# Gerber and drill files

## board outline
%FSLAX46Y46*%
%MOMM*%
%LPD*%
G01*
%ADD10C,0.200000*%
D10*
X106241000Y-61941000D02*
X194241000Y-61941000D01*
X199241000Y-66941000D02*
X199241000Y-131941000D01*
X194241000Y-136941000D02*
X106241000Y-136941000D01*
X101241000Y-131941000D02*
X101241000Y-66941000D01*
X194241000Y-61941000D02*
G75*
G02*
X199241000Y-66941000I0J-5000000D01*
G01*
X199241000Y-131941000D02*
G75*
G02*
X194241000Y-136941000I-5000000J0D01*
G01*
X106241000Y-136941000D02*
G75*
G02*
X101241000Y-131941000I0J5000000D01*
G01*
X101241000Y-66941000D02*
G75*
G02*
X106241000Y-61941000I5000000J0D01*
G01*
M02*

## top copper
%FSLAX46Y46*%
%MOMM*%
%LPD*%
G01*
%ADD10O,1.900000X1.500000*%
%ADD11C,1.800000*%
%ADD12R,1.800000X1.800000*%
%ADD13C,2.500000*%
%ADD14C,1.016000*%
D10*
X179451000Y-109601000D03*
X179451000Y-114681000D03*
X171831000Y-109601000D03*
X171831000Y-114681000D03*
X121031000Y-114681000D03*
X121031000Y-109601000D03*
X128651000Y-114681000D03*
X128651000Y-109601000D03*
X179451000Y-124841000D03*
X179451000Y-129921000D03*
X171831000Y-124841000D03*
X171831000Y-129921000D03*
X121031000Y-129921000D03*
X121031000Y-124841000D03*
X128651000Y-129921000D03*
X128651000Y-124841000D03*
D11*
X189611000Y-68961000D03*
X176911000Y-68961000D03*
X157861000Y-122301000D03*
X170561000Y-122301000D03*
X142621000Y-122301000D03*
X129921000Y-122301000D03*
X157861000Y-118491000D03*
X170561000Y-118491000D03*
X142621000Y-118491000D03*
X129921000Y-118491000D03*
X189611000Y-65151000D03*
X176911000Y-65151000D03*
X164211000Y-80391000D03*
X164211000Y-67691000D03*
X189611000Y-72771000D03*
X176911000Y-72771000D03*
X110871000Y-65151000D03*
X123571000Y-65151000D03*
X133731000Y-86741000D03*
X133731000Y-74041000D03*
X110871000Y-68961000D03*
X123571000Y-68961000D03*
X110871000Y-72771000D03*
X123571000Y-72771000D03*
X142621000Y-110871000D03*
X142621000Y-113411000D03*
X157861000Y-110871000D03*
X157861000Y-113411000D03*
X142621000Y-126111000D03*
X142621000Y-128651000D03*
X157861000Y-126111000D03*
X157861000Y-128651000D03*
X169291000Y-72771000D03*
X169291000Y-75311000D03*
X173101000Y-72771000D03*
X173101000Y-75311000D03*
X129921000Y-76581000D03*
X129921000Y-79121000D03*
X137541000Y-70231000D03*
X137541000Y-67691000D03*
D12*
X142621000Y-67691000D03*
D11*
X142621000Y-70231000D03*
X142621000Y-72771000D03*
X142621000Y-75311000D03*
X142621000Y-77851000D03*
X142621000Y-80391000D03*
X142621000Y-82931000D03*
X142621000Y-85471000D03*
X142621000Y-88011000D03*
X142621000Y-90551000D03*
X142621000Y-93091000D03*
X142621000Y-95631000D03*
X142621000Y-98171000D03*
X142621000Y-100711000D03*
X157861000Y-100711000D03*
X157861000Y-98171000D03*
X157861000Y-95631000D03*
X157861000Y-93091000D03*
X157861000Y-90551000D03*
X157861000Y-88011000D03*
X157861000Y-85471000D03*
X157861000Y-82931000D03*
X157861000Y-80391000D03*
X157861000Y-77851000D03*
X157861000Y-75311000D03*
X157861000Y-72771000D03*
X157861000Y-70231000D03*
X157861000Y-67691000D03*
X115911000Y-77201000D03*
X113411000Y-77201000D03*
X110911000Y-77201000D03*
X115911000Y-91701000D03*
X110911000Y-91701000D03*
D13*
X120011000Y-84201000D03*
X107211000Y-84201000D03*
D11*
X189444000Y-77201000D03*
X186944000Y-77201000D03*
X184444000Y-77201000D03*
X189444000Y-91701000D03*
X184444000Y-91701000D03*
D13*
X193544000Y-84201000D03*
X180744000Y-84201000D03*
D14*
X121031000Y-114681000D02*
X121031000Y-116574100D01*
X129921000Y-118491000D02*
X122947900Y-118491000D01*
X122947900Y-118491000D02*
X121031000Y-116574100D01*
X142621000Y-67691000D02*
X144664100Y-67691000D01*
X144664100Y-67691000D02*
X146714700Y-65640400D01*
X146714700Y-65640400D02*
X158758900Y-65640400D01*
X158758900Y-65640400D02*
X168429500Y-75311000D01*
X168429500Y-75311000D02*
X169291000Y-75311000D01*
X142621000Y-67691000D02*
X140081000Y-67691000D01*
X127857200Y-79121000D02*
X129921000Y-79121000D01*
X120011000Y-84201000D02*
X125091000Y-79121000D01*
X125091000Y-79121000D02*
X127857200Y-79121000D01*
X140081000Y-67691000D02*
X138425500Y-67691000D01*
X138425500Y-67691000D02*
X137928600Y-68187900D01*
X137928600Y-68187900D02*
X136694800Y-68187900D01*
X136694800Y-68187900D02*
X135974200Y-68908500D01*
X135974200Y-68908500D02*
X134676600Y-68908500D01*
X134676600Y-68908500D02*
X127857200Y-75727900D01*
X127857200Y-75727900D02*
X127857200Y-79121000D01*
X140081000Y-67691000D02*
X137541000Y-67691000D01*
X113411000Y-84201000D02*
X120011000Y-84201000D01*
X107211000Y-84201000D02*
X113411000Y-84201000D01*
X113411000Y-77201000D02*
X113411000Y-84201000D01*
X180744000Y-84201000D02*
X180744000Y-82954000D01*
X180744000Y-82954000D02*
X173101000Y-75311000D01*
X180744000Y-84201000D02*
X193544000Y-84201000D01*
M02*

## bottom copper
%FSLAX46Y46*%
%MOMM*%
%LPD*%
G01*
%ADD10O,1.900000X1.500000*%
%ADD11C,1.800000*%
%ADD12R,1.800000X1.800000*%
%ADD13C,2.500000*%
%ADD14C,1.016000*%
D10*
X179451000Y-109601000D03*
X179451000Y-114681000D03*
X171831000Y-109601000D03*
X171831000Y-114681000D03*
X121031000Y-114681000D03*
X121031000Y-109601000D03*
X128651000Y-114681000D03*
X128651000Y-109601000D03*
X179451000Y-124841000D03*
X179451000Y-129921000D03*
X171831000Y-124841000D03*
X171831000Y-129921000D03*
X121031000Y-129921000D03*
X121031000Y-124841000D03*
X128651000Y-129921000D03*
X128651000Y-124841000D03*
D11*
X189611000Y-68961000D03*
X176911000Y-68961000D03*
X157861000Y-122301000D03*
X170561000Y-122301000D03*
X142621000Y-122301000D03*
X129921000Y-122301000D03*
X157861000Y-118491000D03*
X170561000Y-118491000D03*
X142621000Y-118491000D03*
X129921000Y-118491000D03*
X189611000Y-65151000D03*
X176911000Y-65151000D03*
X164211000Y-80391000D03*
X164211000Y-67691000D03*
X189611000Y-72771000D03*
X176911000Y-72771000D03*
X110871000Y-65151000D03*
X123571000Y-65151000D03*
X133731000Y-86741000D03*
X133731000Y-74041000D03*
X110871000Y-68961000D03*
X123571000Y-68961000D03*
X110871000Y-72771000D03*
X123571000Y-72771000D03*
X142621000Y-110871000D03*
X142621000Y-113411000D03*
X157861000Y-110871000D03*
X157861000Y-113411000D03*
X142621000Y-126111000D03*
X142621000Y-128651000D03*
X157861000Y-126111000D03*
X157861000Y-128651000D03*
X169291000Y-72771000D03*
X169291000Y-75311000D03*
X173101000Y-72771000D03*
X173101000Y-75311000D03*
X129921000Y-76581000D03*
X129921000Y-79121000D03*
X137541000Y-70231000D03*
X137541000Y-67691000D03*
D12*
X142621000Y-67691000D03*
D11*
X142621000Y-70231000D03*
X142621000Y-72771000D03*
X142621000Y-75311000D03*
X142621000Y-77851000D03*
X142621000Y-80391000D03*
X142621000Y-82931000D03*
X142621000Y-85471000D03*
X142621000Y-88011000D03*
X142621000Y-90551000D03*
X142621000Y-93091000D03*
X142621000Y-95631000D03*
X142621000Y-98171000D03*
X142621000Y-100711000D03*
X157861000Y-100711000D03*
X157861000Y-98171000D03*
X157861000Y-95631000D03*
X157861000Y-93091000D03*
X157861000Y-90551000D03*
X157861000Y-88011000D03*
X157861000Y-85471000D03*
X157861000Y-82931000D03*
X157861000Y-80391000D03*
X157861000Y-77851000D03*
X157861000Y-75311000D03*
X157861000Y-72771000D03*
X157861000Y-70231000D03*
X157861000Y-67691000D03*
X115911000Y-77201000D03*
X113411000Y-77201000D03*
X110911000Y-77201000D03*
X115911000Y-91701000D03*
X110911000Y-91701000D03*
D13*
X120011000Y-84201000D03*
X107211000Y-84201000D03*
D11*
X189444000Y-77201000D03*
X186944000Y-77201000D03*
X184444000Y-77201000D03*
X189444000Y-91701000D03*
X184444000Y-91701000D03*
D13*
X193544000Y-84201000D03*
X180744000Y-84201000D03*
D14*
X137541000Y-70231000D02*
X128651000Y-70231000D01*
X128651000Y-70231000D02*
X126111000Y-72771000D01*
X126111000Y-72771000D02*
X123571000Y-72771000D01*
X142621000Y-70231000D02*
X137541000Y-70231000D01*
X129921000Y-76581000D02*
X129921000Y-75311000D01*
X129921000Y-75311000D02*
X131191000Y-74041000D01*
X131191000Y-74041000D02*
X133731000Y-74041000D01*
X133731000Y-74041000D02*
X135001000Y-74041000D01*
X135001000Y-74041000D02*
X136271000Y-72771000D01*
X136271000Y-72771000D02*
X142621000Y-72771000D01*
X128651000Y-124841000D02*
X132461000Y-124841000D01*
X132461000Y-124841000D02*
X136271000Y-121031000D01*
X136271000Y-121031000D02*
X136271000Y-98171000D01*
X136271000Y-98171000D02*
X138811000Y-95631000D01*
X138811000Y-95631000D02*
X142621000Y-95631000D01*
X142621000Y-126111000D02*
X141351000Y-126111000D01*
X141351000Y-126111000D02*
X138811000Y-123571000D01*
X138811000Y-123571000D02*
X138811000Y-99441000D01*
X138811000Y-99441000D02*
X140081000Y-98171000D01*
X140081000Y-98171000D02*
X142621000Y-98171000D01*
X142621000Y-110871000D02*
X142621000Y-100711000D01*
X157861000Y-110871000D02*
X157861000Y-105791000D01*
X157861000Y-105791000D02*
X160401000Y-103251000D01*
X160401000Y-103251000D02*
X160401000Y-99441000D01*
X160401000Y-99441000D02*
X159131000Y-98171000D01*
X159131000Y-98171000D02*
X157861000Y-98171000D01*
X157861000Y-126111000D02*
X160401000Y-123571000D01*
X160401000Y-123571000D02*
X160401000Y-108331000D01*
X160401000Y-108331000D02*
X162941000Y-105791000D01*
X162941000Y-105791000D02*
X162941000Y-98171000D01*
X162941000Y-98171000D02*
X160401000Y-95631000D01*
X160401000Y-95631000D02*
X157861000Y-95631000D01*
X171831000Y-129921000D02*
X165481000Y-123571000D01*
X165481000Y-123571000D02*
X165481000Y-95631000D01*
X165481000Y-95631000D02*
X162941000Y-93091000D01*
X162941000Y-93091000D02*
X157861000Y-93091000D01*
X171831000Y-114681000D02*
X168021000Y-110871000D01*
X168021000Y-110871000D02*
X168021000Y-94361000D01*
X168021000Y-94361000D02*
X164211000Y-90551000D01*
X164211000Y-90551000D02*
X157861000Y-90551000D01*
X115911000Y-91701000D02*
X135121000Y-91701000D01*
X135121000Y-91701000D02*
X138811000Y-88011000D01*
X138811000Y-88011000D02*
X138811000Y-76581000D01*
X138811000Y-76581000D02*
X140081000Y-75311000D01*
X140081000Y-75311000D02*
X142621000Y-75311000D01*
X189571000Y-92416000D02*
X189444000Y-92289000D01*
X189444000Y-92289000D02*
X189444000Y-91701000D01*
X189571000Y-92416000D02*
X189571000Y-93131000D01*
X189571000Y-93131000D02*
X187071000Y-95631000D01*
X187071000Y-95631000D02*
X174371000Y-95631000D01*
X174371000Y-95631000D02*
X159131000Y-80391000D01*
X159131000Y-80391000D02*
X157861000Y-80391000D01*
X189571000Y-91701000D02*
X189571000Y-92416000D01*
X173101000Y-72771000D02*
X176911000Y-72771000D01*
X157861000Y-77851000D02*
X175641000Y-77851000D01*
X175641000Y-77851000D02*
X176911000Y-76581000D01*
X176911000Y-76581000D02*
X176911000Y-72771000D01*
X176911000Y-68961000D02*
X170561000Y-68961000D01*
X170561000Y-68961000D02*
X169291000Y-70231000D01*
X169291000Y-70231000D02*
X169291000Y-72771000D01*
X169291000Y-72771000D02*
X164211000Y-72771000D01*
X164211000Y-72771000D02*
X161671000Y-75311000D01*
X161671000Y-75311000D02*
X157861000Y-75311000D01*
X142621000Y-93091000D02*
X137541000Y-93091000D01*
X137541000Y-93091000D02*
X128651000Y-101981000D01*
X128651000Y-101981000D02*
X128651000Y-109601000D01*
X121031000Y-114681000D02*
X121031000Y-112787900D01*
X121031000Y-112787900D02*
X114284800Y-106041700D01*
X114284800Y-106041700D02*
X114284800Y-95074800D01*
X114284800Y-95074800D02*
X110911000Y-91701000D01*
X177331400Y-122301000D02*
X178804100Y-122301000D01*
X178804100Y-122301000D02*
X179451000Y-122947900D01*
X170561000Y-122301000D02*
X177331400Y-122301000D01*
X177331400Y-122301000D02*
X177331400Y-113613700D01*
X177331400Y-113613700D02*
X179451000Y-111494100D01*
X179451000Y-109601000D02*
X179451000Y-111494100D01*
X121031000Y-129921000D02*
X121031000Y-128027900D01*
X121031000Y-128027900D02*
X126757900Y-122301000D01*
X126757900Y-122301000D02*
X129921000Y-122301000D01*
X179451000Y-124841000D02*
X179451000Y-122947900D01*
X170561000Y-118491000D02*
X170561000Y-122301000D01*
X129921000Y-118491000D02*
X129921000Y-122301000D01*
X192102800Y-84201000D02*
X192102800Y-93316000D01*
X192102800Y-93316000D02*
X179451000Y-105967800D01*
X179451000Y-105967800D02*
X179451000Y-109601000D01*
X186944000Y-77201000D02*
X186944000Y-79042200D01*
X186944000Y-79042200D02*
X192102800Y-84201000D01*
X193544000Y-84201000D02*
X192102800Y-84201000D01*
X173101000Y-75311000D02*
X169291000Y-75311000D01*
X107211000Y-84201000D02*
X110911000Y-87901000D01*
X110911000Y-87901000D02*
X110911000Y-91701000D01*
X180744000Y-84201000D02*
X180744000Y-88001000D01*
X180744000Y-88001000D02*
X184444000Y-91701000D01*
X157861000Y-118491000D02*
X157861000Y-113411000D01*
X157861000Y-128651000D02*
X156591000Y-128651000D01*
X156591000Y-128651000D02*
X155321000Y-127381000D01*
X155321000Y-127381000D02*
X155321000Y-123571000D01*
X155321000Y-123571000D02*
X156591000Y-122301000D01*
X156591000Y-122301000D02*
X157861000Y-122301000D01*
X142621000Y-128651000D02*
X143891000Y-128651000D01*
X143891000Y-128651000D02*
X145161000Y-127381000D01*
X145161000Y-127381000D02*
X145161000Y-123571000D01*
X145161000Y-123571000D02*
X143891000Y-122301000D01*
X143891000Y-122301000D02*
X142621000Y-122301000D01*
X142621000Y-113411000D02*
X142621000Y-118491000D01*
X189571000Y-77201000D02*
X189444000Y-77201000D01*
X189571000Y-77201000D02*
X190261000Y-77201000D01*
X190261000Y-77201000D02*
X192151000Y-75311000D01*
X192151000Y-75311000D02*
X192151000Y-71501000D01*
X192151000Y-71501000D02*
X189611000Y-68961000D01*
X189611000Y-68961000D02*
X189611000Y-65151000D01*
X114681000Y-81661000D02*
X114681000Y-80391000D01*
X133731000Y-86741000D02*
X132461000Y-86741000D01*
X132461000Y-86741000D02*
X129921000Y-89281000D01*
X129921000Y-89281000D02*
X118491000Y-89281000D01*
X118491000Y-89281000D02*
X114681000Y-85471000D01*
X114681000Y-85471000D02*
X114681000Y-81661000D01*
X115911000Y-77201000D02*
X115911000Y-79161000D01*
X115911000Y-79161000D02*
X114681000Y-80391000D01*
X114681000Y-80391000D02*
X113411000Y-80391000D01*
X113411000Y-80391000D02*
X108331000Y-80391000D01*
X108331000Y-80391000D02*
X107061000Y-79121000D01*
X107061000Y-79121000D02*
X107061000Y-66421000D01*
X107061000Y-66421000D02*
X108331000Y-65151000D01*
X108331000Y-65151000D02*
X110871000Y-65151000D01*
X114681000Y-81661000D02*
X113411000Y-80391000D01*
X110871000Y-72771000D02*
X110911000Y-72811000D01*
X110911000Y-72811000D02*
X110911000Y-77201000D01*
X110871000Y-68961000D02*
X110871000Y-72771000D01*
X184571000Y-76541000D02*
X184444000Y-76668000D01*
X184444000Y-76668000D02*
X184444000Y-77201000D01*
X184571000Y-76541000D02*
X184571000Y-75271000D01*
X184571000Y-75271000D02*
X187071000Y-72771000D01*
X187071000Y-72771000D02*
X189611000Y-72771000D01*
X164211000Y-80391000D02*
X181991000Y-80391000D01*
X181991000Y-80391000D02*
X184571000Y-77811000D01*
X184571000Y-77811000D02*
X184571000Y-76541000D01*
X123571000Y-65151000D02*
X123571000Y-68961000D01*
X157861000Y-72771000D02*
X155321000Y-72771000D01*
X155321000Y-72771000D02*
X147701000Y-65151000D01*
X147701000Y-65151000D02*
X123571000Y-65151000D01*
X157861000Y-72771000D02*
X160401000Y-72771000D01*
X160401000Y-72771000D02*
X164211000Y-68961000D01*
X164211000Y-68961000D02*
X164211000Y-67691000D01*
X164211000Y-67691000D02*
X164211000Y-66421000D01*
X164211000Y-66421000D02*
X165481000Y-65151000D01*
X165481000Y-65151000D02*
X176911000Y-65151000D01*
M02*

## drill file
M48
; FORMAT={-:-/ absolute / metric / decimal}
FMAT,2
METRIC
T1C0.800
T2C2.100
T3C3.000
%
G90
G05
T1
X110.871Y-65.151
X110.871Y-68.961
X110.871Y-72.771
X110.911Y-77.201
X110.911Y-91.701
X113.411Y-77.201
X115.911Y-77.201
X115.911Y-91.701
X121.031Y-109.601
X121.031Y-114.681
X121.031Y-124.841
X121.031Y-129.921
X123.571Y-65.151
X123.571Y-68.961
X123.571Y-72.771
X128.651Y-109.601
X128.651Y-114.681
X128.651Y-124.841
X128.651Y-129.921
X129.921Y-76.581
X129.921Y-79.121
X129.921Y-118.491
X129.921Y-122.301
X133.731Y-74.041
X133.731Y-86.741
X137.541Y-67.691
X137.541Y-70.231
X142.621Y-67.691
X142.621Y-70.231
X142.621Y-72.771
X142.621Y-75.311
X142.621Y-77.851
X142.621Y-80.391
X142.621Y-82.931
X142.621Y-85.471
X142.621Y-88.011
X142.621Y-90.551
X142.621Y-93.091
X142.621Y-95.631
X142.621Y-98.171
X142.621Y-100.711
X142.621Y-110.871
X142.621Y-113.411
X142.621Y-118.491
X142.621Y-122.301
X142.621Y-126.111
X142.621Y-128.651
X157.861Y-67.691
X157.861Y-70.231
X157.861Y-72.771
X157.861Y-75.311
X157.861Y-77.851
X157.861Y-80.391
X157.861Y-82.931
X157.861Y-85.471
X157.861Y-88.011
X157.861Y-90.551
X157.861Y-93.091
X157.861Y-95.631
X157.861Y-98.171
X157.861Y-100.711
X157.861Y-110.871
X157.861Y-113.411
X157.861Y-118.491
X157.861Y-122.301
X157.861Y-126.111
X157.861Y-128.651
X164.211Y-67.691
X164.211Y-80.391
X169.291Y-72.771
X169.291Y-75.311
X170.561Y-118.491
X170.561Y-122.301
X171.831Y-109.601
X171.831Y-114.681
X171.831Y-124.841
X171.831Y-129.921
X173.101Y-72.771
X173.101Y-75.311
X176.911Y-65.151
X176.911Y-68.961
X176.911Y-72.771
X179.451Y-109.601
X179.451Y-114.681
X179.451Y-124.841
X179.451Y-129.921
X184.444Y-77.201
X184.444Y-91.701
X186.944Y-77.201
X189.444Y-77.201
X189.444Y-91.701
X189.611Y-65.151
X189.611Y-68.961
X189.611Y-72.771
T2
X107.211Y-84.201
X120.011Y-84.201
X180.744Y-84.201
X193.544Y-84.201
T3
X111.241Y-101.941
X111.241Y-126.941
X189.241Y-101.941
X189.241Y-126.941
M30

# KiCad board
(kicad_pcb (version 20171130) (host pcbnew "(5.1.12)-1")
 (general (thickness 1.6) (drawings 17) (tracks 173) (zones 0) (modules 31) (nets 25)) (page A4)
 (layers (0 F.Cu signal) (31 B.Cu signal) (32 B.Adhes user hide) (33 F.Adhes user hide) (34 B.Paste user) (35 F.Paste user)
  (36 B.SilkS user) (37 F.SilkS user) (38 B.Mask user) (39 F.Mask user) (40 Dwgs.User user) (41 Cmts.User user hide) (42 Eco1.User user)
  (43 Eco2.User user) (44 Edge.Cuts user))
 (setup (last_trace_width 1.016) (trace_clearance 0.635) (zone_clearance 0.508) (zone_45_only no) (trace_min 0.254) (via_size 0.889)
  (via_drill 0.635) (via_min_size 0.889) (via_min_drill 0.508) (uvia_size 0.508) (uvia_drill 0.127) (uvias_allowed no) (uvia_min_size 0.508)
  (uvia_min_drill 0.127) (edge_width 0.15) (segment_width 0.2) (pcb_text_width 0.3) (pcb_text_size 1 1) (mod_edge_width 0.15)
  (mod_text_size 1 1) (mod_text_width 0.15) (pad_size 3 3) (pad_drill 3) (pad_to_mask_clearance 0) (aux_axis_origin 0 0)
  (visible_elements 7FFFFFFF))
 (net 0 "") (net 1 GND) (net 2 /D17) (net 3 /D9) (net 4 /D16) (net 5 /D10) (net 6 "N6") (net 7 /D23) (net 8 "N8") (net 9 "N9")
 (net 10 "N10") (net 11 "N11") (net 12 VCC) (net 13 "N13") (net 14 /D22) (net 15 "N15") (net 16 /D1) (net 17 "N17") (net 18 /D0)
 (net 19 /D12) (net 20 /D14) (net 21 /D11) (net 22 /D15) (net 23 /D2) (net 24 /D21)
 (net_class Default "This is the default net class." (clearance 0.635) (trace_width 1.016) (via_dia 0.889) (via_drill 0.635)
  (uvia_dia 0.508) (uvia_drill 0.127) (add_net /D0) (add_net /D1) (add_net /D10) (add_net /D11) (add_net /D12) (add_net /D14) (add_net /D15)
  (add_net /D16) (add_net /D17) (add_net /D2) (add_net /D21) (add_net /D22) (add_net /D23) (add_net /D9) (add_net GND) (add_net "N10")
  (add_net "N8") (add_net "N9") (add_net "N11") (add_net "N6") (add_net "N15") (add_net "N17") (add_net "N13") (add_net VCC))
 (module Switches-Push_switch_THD (layer F.Cu) (at 175.641 112.141 180)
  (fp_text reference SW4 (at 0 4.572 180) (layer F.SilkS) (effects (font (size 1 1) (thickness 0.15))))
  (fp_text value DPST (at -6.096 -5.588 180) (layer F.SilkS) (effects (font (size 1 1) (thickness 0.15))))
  (pad 2 thru_hole oval (at -3.81 2.54 180) (size 1.9 1.5) (drill 0.8) (layers *.Cu *.Mask F.SilkS) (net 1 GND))
  (pad 1 thru_hole oval (at -3.81 -2.54 180) (size 1.9 1.5) (drill 0.8) (layers *.Cu *.Mask F.SilkS))
  (pad 4 thru_hole oval (at 3.81 2.54 180) (size 1.9 1.5) (drill 0.8) (layers *.Cu *.Mask F.SilkS))
  (pad 3 thru_hole oval (at 3.81 -2.54 180) (size 1.9 1.5) (drill 0.8) (layers *.Cu *.Mask F.SilkS) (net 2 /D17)))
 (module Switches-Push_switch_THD (layer F.Cu) (at 124.841 112.141)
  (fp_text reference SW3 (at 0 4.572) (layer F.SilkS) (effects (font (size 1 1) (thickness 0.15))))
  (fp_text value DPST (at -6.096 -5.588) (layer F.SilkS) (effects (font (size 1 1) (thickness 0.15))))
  (pad 2 thru_hole oval (at -3.81 2.54) (size 1.9 1.5) (drill 0.8) (layers *.Cu *.Mask F.SilkS) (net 1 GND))
  (pad 1 thru_hole oval (at -3.81 -2.54) (size 1.9 1.5) (drill 0.8) (layers *.Cu *.Mask F.SilkS))
  (pad 4 thru_hole oval (at 3.81 2.54) (size 1.9 1.5) (drill 0.8) (layers *.Cu *.Mask F.SilkS))
  (pad 3 thru_hole oval (at 3.81 -2.54) (size 1.9 1.5) (drill 0.8) (layers *.Cu *.Mask F.SilkS) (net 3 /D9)))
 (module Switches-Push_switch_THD (layer F.Cu) (at 175.641 127.381 180)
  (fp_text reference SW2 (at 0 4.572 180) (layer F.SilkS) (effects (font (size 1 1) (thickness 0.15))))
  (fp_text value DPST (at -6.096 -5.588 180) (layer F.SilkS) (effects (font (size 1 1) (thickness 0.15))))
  (pad 2 thru_hole oval (at -3.81 2.54 180) (size 1.9 1.5) (drill 0.8) (layers *.Cu *.Mask F.SilkS) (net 1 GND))
  (pad 1 thru_hole oval (at -3.81 -2.54 180) (size 1.9 1.5) (drill 0.8) (layers *.Cu *.Mask F.SilkS))
  (pad 4 thru_hole oval (at 3.81 2.54 180) (size 1.9 1.5) (drill 0.8) (layers *.Cu *.Mask F.SilkS))
  (pad 3 thru_hole oval (at 3.81 -2.54 180) (size 1.9 1.5) (drill 0.8) (layers *.Cu *.Mask F.SilkS) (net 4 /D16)))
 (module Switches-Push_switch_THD (layer F.Cu) (at 124.841 127.381)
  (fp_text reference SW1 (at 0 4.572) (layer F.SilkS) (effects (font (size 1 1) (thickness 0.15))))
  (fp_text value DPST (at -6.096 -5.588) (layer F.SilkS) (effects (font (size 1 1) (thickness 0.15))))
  (pad 2 thru_hole oval (at -3.81 2.54) (size 1.9 1.5) (drill 0.8) (layers *.Cu *.Mask F.SilkS) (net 1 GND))
  (pad 1 thru_hole oval (at -3.81 -2.54) (size 1.9 1.5) (drill 0.8) (layers *.Cu *.Mask F.SilkS))
  (pad 4 thru_hole oval (at 3.81 2.54) (size 1.9 1.5) (drill 0.8) (layers *.Cu *.Mask F.SilkS))
  (pad 3 thru_hole oval (at 3.81 -2.54) (size 1.9 1.5) (drill 0.8) (layers *.Cu *.Mask F.SilkS) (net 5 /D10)))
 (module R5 (layer F.Cu) (at 183.261 68.961 180) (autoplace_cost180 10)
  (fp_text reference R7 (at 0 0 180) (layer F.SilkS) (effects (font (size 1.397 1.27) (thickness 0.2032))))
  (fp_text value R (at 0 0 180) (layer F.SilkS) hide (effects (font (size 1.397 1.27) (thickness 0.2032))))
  (pad 1 thru_hole circle (at -6.35 0 180) (size 1.8 1.8) (drill 0.8) (layers *.Cu *.Mask F.SilkS) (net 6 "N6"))
  (pad 2 thru_hole circle (at 6.35 0 180) (size 1.8 1.8) (drill 0.8) (layers *.Cu *.Mask F.SilkS) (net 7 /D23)))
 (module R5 (layer F.Cu) (at 164.211 122.301) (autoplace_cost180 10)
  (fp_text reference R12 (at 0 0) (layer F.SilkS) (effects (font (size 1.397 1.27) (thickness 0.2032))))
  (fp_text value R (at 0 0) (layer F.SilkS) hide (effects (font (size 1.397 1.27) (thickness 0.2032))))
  (pad 1 thru_hole circle (at -6.35 0) (size 1.8 1.8) (drill 0.8) (layers *.Cu *.Mask F.SilkS) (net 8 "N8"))
  (pad 2 thru_hole circle (at 6.35 0) (size 1.8 1.8) (drill 0.8) (layers *.Cu *.Mask F.SilkS) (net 1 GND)))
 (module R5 (layer F.Cu) (at 136.271 122.301 180) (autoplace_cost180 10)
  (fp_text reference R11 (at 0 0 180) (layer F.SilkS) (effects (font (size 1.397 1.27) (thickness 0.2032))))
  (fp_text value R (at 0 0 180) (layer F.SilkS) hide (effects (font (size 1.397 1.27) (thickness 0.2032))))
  (pad 1 thru_hole circle (at -6.35 0 180) (size 1.8 1.8) (drill 0.8) (layers *.Cu *.Mask F.SilkS) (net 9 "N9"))
  (pad 2 thru_hole circle (at 6.35 0 180) (size 1.8 1.8) (drill 0.8) (layers *.Cu *.Mask F.SilkS) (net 1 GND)))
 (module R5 (layer F.Cu) (at 164.211 118.491) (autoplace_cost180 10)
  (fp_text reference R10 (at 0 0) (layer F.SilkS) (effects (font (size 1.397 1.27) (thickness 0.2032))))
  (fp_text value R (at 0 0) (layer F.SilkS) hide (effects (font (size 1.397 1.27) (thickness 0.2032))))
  (pad 1 thru_hole circle (at -6.35 0) (size 1.8 1.8) (drill 0.8) (layers *.Cu *.Mask F.SilkS) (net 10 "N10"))
  (pad 2 thru_hole circle (at 6.35 0) (size 1.8 1.8) (drill 0.8) (layers *.Cu *.Mask F.SilkS) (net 1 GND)))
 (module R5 (layer F.Cu) (at 136.271 118.491 180) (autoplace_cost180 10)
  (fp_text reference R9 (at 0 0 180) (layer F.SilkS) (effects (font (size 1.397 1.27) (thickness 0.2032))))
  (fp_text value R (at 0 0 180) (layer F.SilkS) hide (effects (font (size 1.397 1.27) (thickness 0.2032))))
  (pad 1 thru_hole circle (at -6.35 0 180) (size 1.8 1.8) (drill 0.8) (layers *.Cu *.Mask F.SilkS) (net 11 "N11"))
  (pad 2 thru_hole circle (at 6.35 0 180) (size 1.8 1.8) (drill 0.8) (layers *.Cu *.Mask F.SilkS) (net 1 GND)))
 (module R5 (layer F.Cu) (at 183.261 65.151 180) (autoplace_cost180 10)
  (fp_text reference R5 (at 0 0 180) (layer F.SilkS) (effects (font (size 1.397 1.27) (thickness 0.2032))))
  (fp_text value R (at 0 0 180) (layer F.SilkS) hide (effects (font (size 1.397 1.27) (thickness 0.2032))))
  (pad 1 thru_hole circle (at -6.35 0 180) (size 1.8 1.8) (drill 0.8) (layers *.Cu *.Mask F.SilkS) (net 6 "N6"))
  (pad 2 thru_hole circle (at 6.35 0 180) (size 1.8 1.8) (drill 0.8) (layers *.Cu *.Mask F.SilkS) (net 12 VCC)))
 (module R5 (layer F.Cu) (at 164.211 74.041 90) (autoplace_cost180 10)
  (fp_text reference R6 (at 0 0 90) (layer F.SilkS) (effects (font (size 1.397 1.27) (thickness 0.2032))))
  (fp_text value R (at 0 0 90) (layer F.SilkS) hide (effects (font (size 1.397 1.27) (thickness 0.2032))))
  (pad 1 thru_hole circle (at -6.35 0 90) (size 1.8 1.8) (drill 0.8) (layers *.Cu *.Mask F.SilkS) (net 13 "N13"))
  (pad 2 thru_hole circle (at 6.35 0 90) (size 1.8 1.8) (drill 0.8) (layers *.Cu *.Mask F.SilkS) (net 12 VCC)))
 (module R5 (layer F.Cu) (at 183.261 72.771 180) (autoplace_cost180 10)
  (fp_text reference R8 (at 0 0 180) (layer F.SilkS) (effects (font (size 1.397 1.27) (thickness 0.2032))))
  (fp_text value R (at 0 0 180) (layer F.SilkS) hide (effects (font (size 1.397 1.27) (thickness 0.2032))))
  (pad 1 thru_hole circle (at -6.35 0 180) (size 1.8 1.8) (drill 0.8) (layers *.Cu *.Mask F.SilkS) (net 13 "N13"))
  (pad 2 thru_hole circle (at 6.35 0 180) (size 1.8 1.8) (drill 0.8) (layers *.Cu *.Mask F.SilkS) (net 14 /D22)))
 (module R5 (layer F.Cu) (at 117.221 65.151) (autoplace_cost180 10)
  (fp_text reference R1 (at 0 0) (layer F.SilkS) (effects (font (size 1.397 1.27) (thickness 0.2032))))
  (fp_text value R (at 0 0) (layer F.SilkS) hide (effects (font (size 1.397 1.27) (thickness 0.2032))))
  (pad 1 thru_hole circle (at -6.35 0) (size 1.8 1.8) (drill 0.8) (layers *.Cu *.Mask F.SilkS) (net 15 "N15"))
  (pad 2 thru_hole circle (at 6.35 0) (size 1.8 1.8) (drill 0.8) (layers *.Cu *.Mask F.SilkS) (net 12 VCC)))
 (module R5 (layer F.Cu) (at 133.731 80.391 90) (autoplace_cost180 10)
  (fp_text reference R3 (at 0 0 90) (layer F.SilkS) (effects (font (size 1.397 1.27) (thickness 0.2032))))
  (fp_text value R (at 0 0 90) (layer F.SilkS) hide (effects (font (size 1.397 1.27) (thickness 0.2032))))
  (pad 1 thru_hole circle (at -6.35 0 90) (size 1.8 1.8) (drill 0.8) (layers *.Cu *.Mask F.SilkS) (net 15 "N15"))
  (pad 2 thru_hole circle (at 6.35 0 90) (size 1.8 1.8) (drill 0.8) (layers *.Cu *.Mask F.SilkS) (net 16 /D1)))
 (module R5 (layer F.Cu) (at 117.221 68.961) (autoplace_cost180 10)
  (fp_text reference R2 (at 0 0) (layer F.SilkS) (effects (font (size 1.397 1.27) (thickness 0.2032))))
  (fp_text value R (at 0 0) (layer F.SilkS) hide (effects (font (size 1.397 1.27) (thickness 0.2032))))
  (pad 1 thru_hole circle (at -6.35 0) (size 1.8 1.8) (drill 0.8) (layers *.Cu *.Mask F.SilkS) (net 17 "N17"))
  (pad 2 thru_hole circle (at 6.35 0) (size 1.8 1.8) (drill 0.8) (layers *.Cu *.Mask F.SilkS) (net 12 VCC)))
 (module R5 (layer F.Cu) (at 117.221 72.771) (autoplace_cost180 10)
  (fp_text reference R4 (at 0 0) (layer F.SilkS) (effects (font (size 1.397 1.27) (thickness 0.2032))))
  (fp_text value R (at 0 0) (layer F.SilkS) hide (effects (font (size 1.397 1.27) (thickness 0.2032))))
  (pad 1 thru_hole circle (at -6.35 0) (size 1.8 1.8) (drill 0.8) (layers *.Cu *.Mask F.SilkS) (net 17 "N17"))
  (pad 2 thru_hole circle (at 6.35 0) (size 1.8 1.8) (drill 0.8) (layers *.Cu *.Mask F.SilkS) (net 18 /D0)))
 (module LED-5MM (layer F.Cu) (at 142.621 112.141 270)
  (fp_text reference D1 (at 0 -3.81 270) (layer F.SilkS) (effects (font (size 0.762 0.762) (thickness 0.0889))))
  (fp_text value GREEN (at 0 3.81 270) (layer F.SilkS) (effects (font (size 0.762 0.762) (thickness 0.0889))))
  (pad 1 thru_hole circle (at -1.27 0 270) (size 1.8 1.8) (drill 0.8) (layers *.Cu *.Mask F.SilkS) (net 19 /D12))
  (pad 2 thru_hole circle (at 1.27 0 270) (size 1.8 1.8) (drill 0.8) (layers *.Cu *.Mask F.SilkS) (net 11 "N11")))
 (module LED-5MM (layer F.Cu) (at 157.861 112.141 270)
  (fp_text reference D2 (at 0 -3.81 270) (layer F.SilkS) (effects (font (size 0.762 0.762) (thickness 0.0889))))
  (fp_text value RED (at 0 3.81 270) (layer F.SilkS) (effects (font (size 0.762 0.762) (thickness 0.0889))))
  (pad 1 thru_hole circle (at -1.27 0 270) (size 1.8 1.8) (drill 0.8) (layers *.Cu *.Mask F.SilkS) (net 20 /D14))
  (pad 2 thru_hole circle (at 1.27 0 270) (size 1.8 1.8) (drill 0.8) (layers *.Cu *.Mask F.SilkS) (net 10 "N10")))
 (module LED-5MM (layer F.Cu) (at 142.621 127.381 270)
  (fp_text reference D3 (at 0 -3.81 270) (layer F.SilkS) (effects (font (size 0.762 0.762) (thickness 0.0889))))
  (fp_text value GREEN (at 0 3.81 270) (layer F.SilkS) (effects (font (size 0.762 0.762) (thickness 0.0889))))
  (pad 1 thru_hole circle (at -1.27 0 270) (size 1.8 1.8) (drill 0.8) (layers *.Cu *.Mask F.SilkS) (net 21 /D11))
  (pad 2 thru_hole circle (at 1.27 0 270) (size 1.8 1.8) (drill 0.8) (layers *.Cu *.Mask F.SilkS) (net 9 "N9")))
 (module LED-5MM (layer F.Cu) (at 157.861 127.381 270)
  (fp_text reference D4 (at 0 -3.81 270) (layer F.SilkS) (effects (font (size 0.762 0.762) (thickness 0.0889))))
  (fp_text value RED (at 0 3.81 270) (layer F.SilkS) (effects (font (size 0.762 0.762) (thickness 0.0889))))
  (pad 1 thru_hole circle (at -1.27 0 270) (size 1.8 1.8) (drill 0.8) (layers *.Cu *.Mask F.SilkS) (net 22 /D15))
  (pad 2 thru_hole circle (at 1.27 0 270) (size 1.8 1.8) (drill 0.8) (layers *.Cu *.Mask F.SilkS) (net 8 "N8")))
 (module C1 (layer F.Cu) (at 169.291 74.041 270)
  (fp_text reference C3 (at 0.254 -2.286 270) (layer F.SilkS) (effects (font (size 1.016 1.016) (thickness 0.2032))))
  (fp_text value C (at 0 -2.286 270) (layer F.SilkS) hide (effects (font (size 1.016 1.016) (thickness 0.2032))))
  (pad 1 thru_hole circle (at -1.27 0 270) (size 1.8 1.8) (drill 0.8) (layers *.Cu *.Mask F.SilkS) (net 7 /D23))
  (pad 2 thru_hole circle (at 1.27 0 270) (size 1.8 1.8) (drill 0.8) (layers *.Cu *.Mask F.SilkS) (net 1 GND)))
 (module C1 (layer F.Cu) (at 173.101 74.041 270)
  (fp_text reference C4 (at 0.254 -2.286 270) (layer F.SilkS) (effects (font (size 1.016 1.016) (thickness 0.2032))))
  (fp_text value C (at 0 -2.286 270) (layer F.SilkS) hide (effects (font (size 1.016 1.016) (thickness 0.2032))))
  (pad 1 thru_hole circle (at -1.27 0 270) (size 1.8 1.8) (drill 0.8) (layers *.Cu *.Mask F.SilkS) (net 14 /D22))
  (pad 2 thru_hole circle (at 1.27 0 270) (size 1.8 1.8) (drill 0.8) (layers *.Cu *.Mask F.SilkS) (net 1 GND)))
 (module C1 (layer F.Cu) (at 129.921 77.851 270)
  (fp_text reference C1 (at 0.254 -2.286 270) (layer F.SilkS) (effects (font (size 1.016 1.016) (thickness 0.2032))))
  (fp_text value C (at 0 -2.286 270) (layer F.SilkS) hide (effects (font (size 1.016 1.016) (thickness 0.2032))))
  (pad 1 thru_hole circle (at -1.27 0 270) (size 1.8 1.8) (drill 0.8) (layers *.Cu *.Mask F.SilkS) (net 16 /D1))
  (pad 2 thru_hole circle (at 1.27 0 270) (size 1.8 1.8) (drill 0.8) (layers *.Cu *.Mask F.SilkS) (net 1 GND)))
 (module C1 (layer F.Cu) (at 137.541 68.961 90)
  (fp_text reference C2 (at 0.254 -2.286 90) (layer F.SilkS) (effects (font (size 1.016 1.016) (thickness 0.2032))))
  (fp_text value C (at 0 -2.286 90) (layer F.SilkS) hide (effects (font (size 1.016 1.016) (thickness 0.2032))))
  (pad 1 thru_hole circle (at -1.27 0 90) (size 1.8 1.8) (drill 0.8) (layers *.Cu *.Mask F.SilkS) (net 18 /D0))
  (pad 2 thru_hole circle (at 1.27 0 90) (size 1.8 1.8) (drill 0.8) (layers *.Cu *.Mask F.SilkS) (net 1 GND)))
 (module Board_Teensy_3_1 (layer F.Cu) (at 150.241 85.471)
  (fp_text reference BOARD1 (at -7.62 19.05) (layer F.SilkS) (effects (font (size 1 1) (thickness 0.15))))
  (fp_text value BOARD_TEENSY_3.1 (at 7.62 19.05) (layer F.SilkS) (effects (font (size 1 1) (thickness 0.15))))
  (pad 1 thru_hole rect (at -7.62 -17.78) (size 1.8 1.8) (drill 0.8) (layers *.Cu *.Mask F.SilkS) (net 1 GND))
  (pad 2 thru_hole circle (at -7.62 -15.24) (size 1.8 1.8) (drill 0.8) (layers *.Cu *.Mask F.SilkS) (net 18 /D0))
  (pad 3 thru_hole circle (at -7.62 -12.7) (size 1.8 1.8) (drill 0.8) (layers *.Cu *.Mask F.SilkS) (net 16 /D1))
  (pad 4 thru_hole circle (at -7.62 -10.16) (size 1.8 1.8) (drill 0.8) (layers *.Cu *.Mask F.SilkS) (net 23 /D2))
  (pad 5 thru_hole circle (at -7.62 -7.62) (size 1.8 1.8) (drill 0.8) (layers *.Cu *.Mask F.SilkS))
  (pad 6 thru_hole circle (at -7.62 -5.08) (size 1.8 1.8) (drill 0.8) (layers *.Cu *.Mask F.SilkS))
  (pad 7 thru_hole circle (at -7.62 -2.54) (size 1.8 1.8) (drill 0.8) (layers *.Cu *.Mask F.SilkS))
  (pad 8 thru_hole circle (at -7.62 0) (size 1.8 1.8) (drill 0.8) (layers *.Cu *.Mask F.SilkS))
  (pad 9 thru_hole circle (at -7.62 2.54) (size 1.8 1.8) (drill 0.8) (layers *.Cu *.Mask F.SilkS))
  (pad 10 thru_hole circle (at -7.62 5.08) (size 1.8 1.8) (drill 0.8) (layers *.Cu *.Mask F.SilkS))
  (pad 11 thru_hole circle (at -7.62 7.62) (size 1.8 1.8) (drill 0.8) (layers *.Cu *.Mask F.SilkS) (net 3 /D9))
  (pad 12 thru_hole circle (at -7.62 10.16) (size 1.8 1.8) (drill 0.8) (layers *.Cu *.Mask F.SilkS) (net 5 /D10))
  (pad 13 thru_hole circle (at -7.62 12.7) (size 1.8 1.8) (drill 0.8) (layers *.Cu *.Mask F.SilkS) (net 21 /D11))
  (pad 14 thru_hole circle (at -7.62 15.24) (size 1.8 1.8) (drill 0.8) (layers *.Cu *.Mask F.SilkS) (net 19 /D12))
  (pad 15 thru_hole circle (at 7.62 15.24) (size 1.8 1.8) (drill 0.8) (layers *.Cu *.Mask F.SilkS))
  (pad 16 thru_hole circle (at 7.62 12.7) (size 1.8 1.8) (drill 0.8) (layers *.Cu *.Mask F.SilkS) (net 20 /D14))
  (pad 17 thru_hole circle (at 7.62 10.16) (size 1.8 1.8) (drill 0.8) (layers *.Cu *.Mask F.SilkS) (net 22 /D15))
  (pad 18 thru_hole circle (at 7.62 7.62) (size 1.8 1.8) (drill 0.8) (layers *.Cu *.Mask F.SilkS) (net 4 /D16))
  (pad 19 thru_hole circle (at 7.62 5.08) (size 1.8 1.8) (drill 0.8) (layers *.Cu *.Mask F.SilkS) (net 2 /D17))
  (pad 20 thru_hole circle (at 7.62 2.54) (size 1.8 1.8) (drill 0.8) (layers *.Cu *.Mask F.SilkS))
  (pad 21 thru_hole circle (at 7.62 0) (size 1.8 1.8) (drill 0.8) (layers *.Cu *.Mask F.SilkS))
  (pad 22 thru_hole circle (at 7.62 -2.54) (size 1.8 1.8) (drill 0.8) (layers *.Cu *.Mask F.SilkS))
  (pad 23 thru_hole circle (at 7.62 -5.08) (size 1.8 1.8) (drill 0.8) (layers *.Cu *.Mask F.SilkS) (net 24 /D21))
  (pad 24 thru_hole circle (at 7.62 -7.62) (size 1.8 1.8) (drill 0.8) (layers *.Cu *.Mask F.SilkS) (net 14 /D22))
  (pad 25 thru_hole circle (at 7.62 -10.16) (size 1.8 1.8) (drill 0.8) (layers *.Cu *.Mask F.SilkS) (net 7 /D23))
  (pad 26 thru_hole circle (at 7.62 -12.7) (size 1.8 1.8) (drill 0.8) (layers *.Cu *.Mask F.SilkS) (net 12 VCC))
  (pad 27 thru_hole circle (at 7.62 -15.24) (size 1.8 1.8) (drill 0.8) (layers *.Cu *.Mask F.SilkS))
  (pad 28 thru_hole circle (at 7.62 -17.78) (size 1.8 1.8) (drill 0.8) (layers *.Cu *.Mask F.SilkS)))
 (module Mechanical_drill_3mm (layer F.Cu) (at 107.95 130.81)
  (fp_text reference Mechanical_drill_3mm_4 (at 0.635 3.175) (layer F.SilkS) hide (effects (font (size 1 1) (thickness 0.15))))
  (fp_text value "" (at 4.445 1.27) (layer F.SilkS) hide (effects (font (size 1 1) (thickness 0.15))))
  (pad "" np_thru_hole circle (at 3.291 -3.869) (size 3 3) (drill 3) (layers *.Cu *.Mask)))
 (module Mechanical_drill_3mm (layer F.Cu) (at 193.04 130.81)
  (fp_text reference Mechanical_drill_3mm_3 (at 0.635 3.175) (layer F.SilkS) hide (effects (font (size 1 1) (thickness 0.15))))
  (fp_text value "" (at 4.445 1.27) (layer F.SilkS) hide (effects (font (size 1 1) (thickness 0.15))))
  (pad "" np_thru_hole circle (at -3.799 -3.869) (size 3 3) (drill 3) (layers *.Cu *.Mask)))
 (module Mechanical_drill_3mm (layer F.Cu) (at 191.77 102.87)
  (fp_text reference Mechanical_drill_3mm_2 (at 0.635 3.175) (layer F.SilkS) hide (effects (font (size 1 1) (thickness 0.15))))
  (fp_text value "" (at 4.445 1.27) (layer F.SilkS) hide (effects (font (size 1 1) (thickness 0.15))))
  (pad "" np_thru_hole circle (at -2.529 -0.929) (size 3 3) (drill 3) (layers *.Cu *.Mask)))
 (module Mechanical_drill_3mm (layer F.Cu) (at 107.95 101.6)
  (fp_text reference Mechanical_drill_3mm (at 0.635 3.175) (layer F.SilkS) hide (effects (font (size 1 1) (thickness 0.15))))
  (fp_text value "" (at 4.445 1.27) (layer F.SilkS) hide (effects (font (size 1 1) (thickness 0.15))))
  (pad "" np_thru_hole circle (at 3.291 0.341) (size 3 3) (drill 3) (layers *.Cu *.Mask)))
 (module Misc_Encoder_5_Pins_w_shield (layer F.Cu) (at 113.411 84.201 270)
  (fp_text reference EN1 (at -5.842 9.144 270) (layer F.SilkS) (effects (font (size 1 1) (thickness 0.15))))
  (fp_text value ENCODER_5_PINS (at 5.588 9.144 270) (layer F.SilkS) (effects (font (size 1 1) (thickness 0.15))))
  (pad 1 thru_hole circle (at -7 -2.5 270) (size 1.8 1.8) (drill 0.8) (layers *.Cu *.Mask F.SilkS) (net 15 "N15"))
  (pad 2 thru_hole circle (at -7 0 270) (size 1.8 1.8) (drill 0.8) (layers *.Cu *.Mask F.SilkS) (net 1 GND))
  (pad 3 thru_hole circle (at -7 2.5 270) (size 1.8 1.8) (drill 0.8) (layers *.Cu *.Mask F.SilkS) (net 17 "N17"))
  (pad 4 thru_hole circle (at 7.5 -2.5 270) (size 1.8 1.8) (drill 0.8) (layers *.Cu *.Mask F.SilkS) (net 23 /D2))
  (pad 5 thru_hole circle (at 7.5 2.5 270) (size 1.8 1.8) (drill 0.8) (layers *.Cu *.Mask F.SilkS) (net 1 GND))
  (pad SHLD thru_hole circle (at 0 -6.6 270) (size 2.5 2.5) (drill 2.1) (layers *.Cu *.Mask F.SilkS) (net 1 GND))
  (pad SHLD thru_hole circle (at 0 6.2 270) (size 2.5 2.5) (drill 2.1) (layers *.Cu *.Mask F.SilkS) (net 1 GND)))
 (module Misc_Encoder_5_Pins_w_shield (layer F.Cu) (at 186.944 84.201 270)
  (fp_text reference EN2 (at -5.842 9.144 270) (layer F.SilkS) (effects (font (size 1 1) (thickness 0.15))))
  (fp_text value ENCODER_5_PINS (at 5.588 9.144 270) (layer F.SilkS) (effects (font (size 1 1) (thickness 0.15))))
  (pad 1 thru_hole circle (at -7 -2.5 270) (size 1.8 1.8) (drill 0.8) (layers *.Cu *.Mask F.SilkS) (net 6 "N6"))
  (pad 2 thru_hole circle (at -7 0 270) (size 1.8 1.8) (drill 0.8) (layers *.Cu *.Mask F.SilkS) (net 1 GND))
  (pad 3 thru_hole circle (at -7 2.5 270) (size 1.8 1.8) (drill 0.8) (layers *.Cu *.Mask F.SilkS) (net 13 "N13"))
  (pad 4 thru_hole circle (at 7.5 -2.5 270) (size 1.8 1.8) (drill 0.8) (layers *.Cu *.Mask F.SilkS) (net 24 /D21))
  (pad 5 thru_hole circle (at 7.5 2.5 270) (size 1.8 1.8) (drill 0.8) (layers *.Cu *.Mask F.SilkS) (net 1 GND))
  (pad SHLD thru_hole circle (at 0 -6.6 270) (size 2.5 2.5) (drill 2.1) (layers *.Cu *.Mask F.SilkS) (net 1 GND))
  (pad SHLD thru_hole circle (at 0 6.2 270) (size 2.5 2.5) (drill 2.1) (layers *.Cu *.Mask F.SilkS) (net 1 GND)))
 (gr_line (start 106.241 61.941) (end 194.241 61.941) (angle 90) (layer Edge.Cuts) (width 0.2))
 (gr_line (start 199.241 66.941) (end 199.241 131.941) (angle 90) (layer Edge.Cuts) (width 0.2))
 (gr_line (start 194.241 136.941) (end 106.241 136.941) (angle 90) (layer Edge.Cuts) (width 0.2))
 (gr_line (start 101.241 131.941) (end 101.241 66.941) (angle 90) (layer Edge.Cuts) (width 0.2))
 (gr_arc (start 194.241 66.941) (end 194.241 61.941) (angle 90) (layer Edge.Cuts) (width 0.2))
 (gr_arc (start 194.241 131.941) (end 199.241 131.941) (angle 90) (layer Edge.Cuts) (width 0.2))
 (gr_arc (start 106.241 131.941) (end 106.241 136.941) (angle 90) (layer Edge.Cuts) (width 0.2))
 (gr_arc (start 106.241 66.941) (end 101.241 66.941) (angle 90) (layer Edge.Cuts) (width 0.2))
 (segment (start 137.541 70.231) (end 128.651 70.231) (width 1.016) (layer B.Cu) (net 18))
 (segment (start 128.651 70.231) (end 126.111 72.771) (width 1.016) (layer B.Cu) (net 18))
 (segment (start 126.111 72.771) (end 123.571 72.771) (width 1.016) (layer B.Cu) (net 18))
 (segment (start 142.621 70.231) (end 137.541 70.231) (width 1.016) (layer B.Cu) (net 18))
 (segment (start 129.921 76.581) (end 129.921 75.311) (width 1.016) (layer B.Cu) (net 16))
 (segment (start 129.921 75.311) (end 131.191 74.041) (width 1.016) (layer B.Cu) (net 16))
 (segment (start 131.191 74.041) (end 133.731 74.041) (width 1.016) (layer B.Cu) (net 16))
 (segment (start 133.731 74.041) (end 135.001 74.041) (width 1.016) (layer B.Cu) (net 16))
 (segment (start 135.001 74.041) (end 136.271 72.771) (width 1.016) (layer B.Cu) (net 16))
 (segment (start 136.271 72.771) (end 142.621 72.771) (width 1.016) (layer B.Cu) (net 16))
 (segment (start 128.651 124.841) (end 132.461 124.841) (width 1.016) (layer B.Cu) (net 5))
 (segment (start 132.461 124.841) (end 136.271 121.031) (width 1.016) (layer B.Cu) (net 5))
 (segment (start 136.271 121.031) (end 136.271 98.171) (width 1.016) (layer B.Cu) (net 5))
 (segment (start 136.271 98.171) (end 138.811 95.631) (width 1.016) (layer B.Cu) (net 5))
 (segment (start 138.811 95.631) (end 142.621 95.631) (width 1.016) (layer B.Cu) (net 5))
 (segment (start 142.621 126.111) (end 141.351 126.111) (width 1.016) (layer B.Cu) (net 21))
 (segment (start 141.351 126.111) (end 138.811 123.571) (width 1.016) (layer B.Cu) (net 21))
 (segment (start 138.811 123.571) (end 138.811 99.441) (width 1.016) (layer B.Cu) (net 21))
 (segment (start 138.811 99.441) (end 140.081 98.171) (width 1.016) (layer B.Cu) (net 21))
 (segment (start 140.081 98.171) (end 142.621 98.171) (width 1.016) (layer B.Cu) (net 21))
 (segment (start 142.621 110.871) (end 142.621 100.711) (width 1.016) (layer B.Cu) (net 19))
 (segment (start 157.861 110.871) (end 157.861 105.791) (width 1.016) (layer B.Cu) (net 20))
 (segment (start 157.861 105.791) (end 160.401 103.251) (width 1.016) (layer B.Cu) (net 20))
 (segment (start 160.401 103.251) (end 160.401 99.441) (width 1.016) (layer B.Cu) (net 20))
 (segment (start 160.401 99.441) (end 159.131 98.171) (width 1.016) (layer B.Cu) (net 20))
 (segment (start 159.131 98.171) (end 157.861 98.171) (width 1.016) (layer B.Cu) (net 20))
 (segment (start 157.861 126.111) (end 160.401 123.571) (width 1.016) (layer B.Cu) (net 22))
 (segment (start 160.401 123.571) (end 160.401 108.331) (width 1.016) (layer B.Cu) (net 22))
 (segment (start 160.401 108.331) (end 162.941 105.791) (width 1.016) (layer B.Cu) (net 22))
 (segment (start 162.941 105.791) (end 162.941 98.171) (width 1.016) (layer B.Cu) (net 22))
 (segment (start 162.941 98.171) (end 160.401 95.631) (width 1.016) (layer B.Cu) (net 22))
 (segment (start 160.401 95.631) (end 157.861 95.631) (width 1.016) (layer B.Cu) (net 22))
 (segment (start 171.831 129.921) (end 165.481 123.571) (width 1.016) (layer B.Cu) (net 4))
 (segment (start 165.481 123.571) (end 165.481 95.631) (width 1.016) (layer B.Cu) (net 4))
 (segment (start 165.481 95.631) (end 162.941 93.091) (width 1.016) (layer B.Cu) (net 4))
 (segment (start 162.941 93.091) (end 157.861 93.091) (width 1.016) (layer B.Cu) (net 4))
 (segment (start 171.831 114.681) (end 168.021 110.871) (width 1.016) (layer B.Cu) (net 2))
 (segment (start 168.021 110.871) (end 168.021 94.361) (width 1.016) (layer B.Cu) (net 2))
 (segment (start 168.021 94.361) (end 164.211 90.551) (width 1.016) (layer B.Cu) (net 2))
 (segment (start 164.211 90.551) (end 157.861 90.551) (width 1.016) (layer B.Cu) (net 2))
 (segment (start 115.911 91.701) (end 135.121 91.701) (width 1.016) (layer B.Cu) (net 23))
 (segment (start 135.121 91.701) (end 138.811 88.011) (width 1.016) (layer B.Cu) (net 23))
 (segment (start 138.811 88.011) (end 138.811 76.581) (width 1.016) (layer B.Cu) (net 23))
 (segment (start 138.811 76.581) (end 140.081 75.311) (width 1.016) (layer B.Cu) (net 23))
 (segment (start 140.081 75.311) (end 142.621 75.311) (width 1.016) (layer B.Cu) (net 23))
 (segment (start 189.571 92.416) (end 189.444 92.289) (width 1.016) (layer B.Cu) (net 24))
 (segment (start 189.444 92.289) (end 189.444 91.701) (width 1.016) (layer B.Cu) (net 24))
 (segment (start 189.571 92.416) (end 189.571 93.131) (width 1.016) (layer B.Cu) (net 24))
 (segment (start 189.571 93.131) (end 187.071 95.631) (width 1.016) (layer B.Cu) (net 24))
 (segment (start 187.071 95.631) (end 174.371 95.631) (width 1.016) (layer B.Cu) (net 24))
 (segment (start 174.371 95.631) (end 159.131 80.391) (width 1.016) (layer B.Cu) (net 24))
 (segment (start 159.131 80.391) (end 157.861 80.391) (width 1.016) (layer B.Cu) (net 24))
 (segment (start 189.571 91.701) (end 189.571 92.416) (width 1.016) (layer B.Cu) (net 24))
 (segment (start 173.101 72.771) (end 176.911 72.771) (width 1.016) (layer B.Cu) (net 14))
 (segment (start 157.861 77.851) (end 175.641 77.851) (width 1.016) (layer B.Cu) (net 14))
 (segment (start 175.641 77.851) (end 176.911 76.581) (width 1.016) (layer B.Cu) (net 14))
 (segment (start 176.911 76.581) (end 176.911 72.771) (width 1.016) (layer B.Cu) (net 14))
 (segment (start 176.911 68.961) (end 170.561 68.961) (width 1.016) (layer B.Cu) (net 7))
 (segment (start 170.561 68.961) (end 169.291 70.231) (width 1.016) (layer B.Cu) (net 7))
 (segment (start 169.291 70.231) (end 169.291 72.771) (width 1.016) (layer B.Cu) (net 7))
 (segment (start 169.291 72.771) (end 164.211 72.771) (width 1.016) (layer B.Cu) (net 7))
 (segment (start 164.211 72.771) (end 161.671 75.311) (width 1.016) (layer B.Cu) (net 7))
 (segment (start 161.671 75.311) (end 157.861 75.311) (width 1.016) (layer B.Cu) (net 7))
 (segment (start 142.621 93.091) (end 137.541 93.091) (width 1.016) (layer B.Cu) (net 3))
 (segment (start 137.541 93.091) (end 128.651 101.981) (width 1.016) (layer B.Cu) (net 3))
 (segment (start 128.651 101.981) (end 128.651 109.601) (width 1.016) (layer B.Cu) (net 3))
 (segment (start 121.031 114.681) (end 121.031 112.7879) (width 1.016) (layer B.Cu) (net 1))
 (segment (start 121.031 112.7879) (end 114.2848 106.0417) (width 1.016) (layer B.Cu) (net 1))
 (segment (start 114.2848 106.0417) (end 114.2848 95.0748) (width 1.016) (layer B.Cu) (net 1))
 (segment (start 114.2848 95.0748) (end 110.911 91.701) (width 1.016) (layer B.Cu) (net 1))
 (segment (start 177.3314 122.301) (end 178.8041 122.301) (width 1.016) (layer B.Cu) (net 1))
 (segment (start 178.8041 122.301) (end 179.451 122.9479) (width 1.016) (layer B.Cu) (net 1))
 (segment (start 170.561 122.301) (end 177.3314 122.301) (width 1.016) (layer B.Cu) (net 1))
 (segment (start 177.3314 122.301) (end 177.3314 113.6137) (width 1.016) (layer B.Cu) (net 1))
 (segment (start 177.3314 113.6137) (end 179.451 111.4941) (width 1.016) (layer B.Cu) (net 1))
 (segment (start 179.451 109.601) (end 179.451 111.4941) (width 1.016) (layer B.Cu) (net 1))
 (segment (start 121.031 129.921) (end 121.031 128.0279) (width 1.016) (layer B.Cu) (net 1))
 (segment (start 121.031 128.0279) (end 126.7579 122.301) (width 1.016) (layer B.Cu) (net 1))
 (segment (start 126.7579 122.301) (end 129.921 122.301) (width 1.016) (layer B.Cu) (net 1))
 (segment (start 179.451 124.841) (end 179.451 122.9479) (width 1.016) (layer B.Cu) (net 1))
 (segment (start 170.561 118.491) (end 170.561 122.301) (width 1.016) (layer B.Cu) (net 1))
 (segment (start 121.031 114.681) (end 121.031 116.5741) (width 1.016) (layer F.Cu) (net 1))
 (segment (start 129.921 118.491) (end 122.9479 118.491) (width 1.016) (layer F.Cu) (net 1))
 (segment (start 122.9479 118.491) (end 121.031 116.5741) (width 1.016) (layer F.Cu) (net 1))
 (segment (start 129.921 118.491) (end 129.921 122.301) (width 1.016) (layer B.Cu) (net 1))
 (segment (start 192.1028 84.201) (end 192.1028 93.316) (width 1.016) (layer B.Cu) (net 1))
 (segment (start 192.1028 93.316) (end 179.451 105.9678) (width 1.016) (layer B.Cu) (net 1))
 (segment (start 179.451 105.9678) (end 179.451 109.601) (width 1.016) (layer B.Cu) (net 1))
 (segment (start 186.944 77.201) (end 186.944 79.0422) (width 1.016) (layer B.Cu) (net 1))
 (segment (start 186.944 79.0422) (end 192.1028 84.201) (width 1.016) (layer B.Cu) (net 1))
 (segment (start 193.544 84.201) (end 192.1028 84.201) (width 1.016) (layer B.Cu) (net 1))
 (segment (start 173.101 75.311) (end 169.291 75.311) (width 1.016) (layer B.Cu) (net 1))
 (segment (start 142.621 67.691) (end 144.6641 67.691) (width 1.016) (layer F.Cu) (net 1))
 (segment (start 144.6641 67.691) (end 146.7147 65.6404) (width 1.016) (layer F.Cu) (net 1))
 (segment (start 146.7147 65.6404) (end 158.7589 65.6404) (width 1.016) (layer F.Cu) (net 1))
 (segment (start 158.7589 65.6404) (end 168.4295 75.311) (width 1.016) (layer F.Cu) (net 1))
 (segment (start 168.4295 75.311) (end 169.291 75.311) (width 1.016) (layer F.Cu) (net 1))
 (segment (start 142.621 67.691) (end 140.081 67.691) (width 1.016) (layer F.Cu) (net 1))
 (segment (start 127.8572 79.121) (end 129.921 79.121) (width 1.016) (layer F.Cu) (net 1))
 (segment (start 120.011 84.201) (end 125.091 79.121) (width 1.016) (layer F.Cu) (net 1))
 (segment (start 125.091 79.121) (end 127.8572 79.121) (width 1.016) (layer F.Cu) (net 1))
 (segment (start 140.081 67.691) (end 138.4255 67.691) (width 1.016) (layer F.Cu) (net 1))
 (segment (start 138.4255 67.691) (end 137.9286 68.1879) (width 1.016) (layer F.Cu) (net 1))
 (segment (start 137.9286 68.1879) (end 136.6948 68.1879) (width 1.016) (layer F.Cu) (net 1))
 (segment (start 136.6948 68.1879) (end 135.9742 68.9085) (width 1.016) (layer F.Cu) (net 1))
 (segment (start 135.9742 68.9085) (end 134.6766 68.9085) (width 1.016) (layer F.Cu) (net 1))
 (segment (start 134.6766 68.9085) (end 127.8572 75.7279) (width 1.016) (layer F.Cu) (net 1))
 (segment (start 127.8572 75.7279) (end 127.8572 79.121) (width 1.016) (layer F.Cu) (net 1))
 (segment (start 140.081 67.691) (end 137.541 67.691) (width 1.016) (layer F.Cu) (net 1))
 (segment (start 113.411 84.201) (end 120.011 84.201) (width 1.016) (layer F.Cu) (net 1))
 (segment (start 107.211 84.201) (end 113.411 84.201) (width 1.016) (layer F.Cu) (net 1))
 (segment (start 113.411 77.201) (end 113.411 84.201) (width 1.016) (layer F.Cu) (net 1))
 (segment (start 107.211 84.201) (end 110.911 87.901) (width 1.016) (layer B.Cu) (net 1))
 (segment (start 110.911 87.901) (end 110.911 91.701) (width 1.016) (layer B.Cu) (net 1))
 (segment (start 180.744 84.201) (end 180.744 82.954) (width 1.016) (layer F.Cu) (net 1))
 (segment (start 180.744 82.954) (end 173.101 75.311) (width 1.016) (layer F.Cu) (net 1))
 (segment (start 180.744 84.201) (end 193.544 84.201) (width 1.016) (layer F.Cu) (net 1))
 (segment (start 180.744 84.201) (end 180.744 88.001) (width 1.016) (layer B.Cu) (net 1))
 (segment (start 180.744 88.001) (end 184.444 91.701) (width 1.016) (layer B.Cu) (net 1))
 (segment (start 157.861 118.491) (end 157.861 113.411) (width 1.016) (layer B.Cu) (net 10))
 (segment (start 157.861 128.651) (end 156.591 128.651) (width 1.016) (layer B.Cu) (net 8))
 (segment (start 156.591 128.651) (end 155.321 127.381) (width 1.016) (layer B.Cu) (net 8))
 (segment (start 155.321 127.381) (end 155.321 123.571) (width 1.016) (layer B.Cu) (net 8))
 (segment (start 155.321 123.571) (end 156.591 122.301) (width 1.016) (layer B.Cu) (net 8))
 (segment (start 156.591 122.301) (end 157.861 122.301) (width 1.016) (layer B.Cu) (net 8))
 (segment (start 142.621 128.651) (end 143.891 128.651) (width 1.016) (layer B.Cu) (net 9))
 (segment (start 143.891 128.651) (end 145.161 127.381) (width 1.016) (layer B.Cu) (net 9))
 (segment (start 145.161 127.381) (end 145.161 123.571) (width 1.016) (layer B.Cu) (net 9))
 (segment (start 145.161 123.571) (end 143.891 122.301) (width 1.016) (layer B.Cu) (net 9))
 (segment (start 143.891 122.301) (end 142.621 122.301) (width 1.016) (layer B.Cu) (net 9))
 (segment (start 142.621 113.411) (end 142.621 118.491) (width 1.016) (layer B.Cu) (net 11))
 (segment (start 189.571 77.201) (end 189.444 77.201) (width 1.016) (layer B.Cu) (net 6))
 (segment (start 189.571 77.201) (end 190.261 77.201) (width 1.016) (layer B.Cu) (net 6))
 (segment (start 190.261 77.201) (end 192.151 75.311) (width 1.016) (layer B.Cu) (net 6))
 (segment (start 192.151 75.311) (end 192.151 71.501) (width 1.016) (layer B.Cu) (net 6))
 (segment (start 192.151 71.501) (end 189.611 68.961) (width 1.016) (layer B.Cu) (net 6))
 (segment (start 189.611 68.961) (end 189.611 65.151) (width 1.016) (layer B.Cu) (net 6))
 (segment (start 114.681 81.661) (end 114.681 80.391) (width 1.016) (layer B.Cu) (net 15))
 (segment (start 133.731 86.741) (end 132.461 86.741) (width 1.016) (layer B.Cu) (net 15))
 (segment (start 132.461 86.741) (end 129.921 89.281) (width 1.016) (layer B.Cu) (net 15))
 (segment (start 129.921 89.281) (end 118.491 89.281) (width 1.016) (layer B.Cu) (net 15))
 (segment (start 118.491 89.281) (end 114.681 85.471) (width 1.016) (layer B.Cu) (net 15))
 (segment (start 114.681 85.471) (end 114.681 81.661) (width 1.016) (layer B.Cu) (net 15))
 (segment (start 115.911 77.201) (end 115.911 79.161) (width 1.016) (layer B.Cu) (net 15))
 (segment (start 115.911 79.161) (end 114.681 80.391) (width 1.016) (layer B.Cu) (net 15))
 (segment (start 114.681 80.391) (end 113.411 80.391) (width 1.016) (layer B.Cu) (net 15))
 (segment (start 113.411 80.391) (end 108.331 80.391) (width 1.016) (layer B.Cu) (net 15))
 (segment (start 108.331 80.391) (end 107.061 79.121) (width 1.016) (layer B.Cu) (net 15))
 (segment (start 107.061 79.121) (end 107.061 66.421) (width 1.016) (layer B.Cu) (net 15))
 (segment (start 107.061 66.421) (end 108.331 65.151) (width 1.016) (layer B.Cu) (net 15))
 (segment (start 108.331 65.151) (end 110.871 65.151) (width 1.016) (layer B.Cu) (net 15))
 (segment (start 114.681 81.661) (end 113.411 80.391) (width 1.016) (layer B.Cu) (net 15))
 (segment (start 110.871 72.771) (end 110.911 72.811) (width 1.016) (layer B.Cu) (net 17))
 (segment (start 110.911 72.811) (end 110.911 77.201) (width 1.016) (layer B.Cu) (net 17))
 (segment (start 110.871 68.961) (end 110.871 72.771) (width 1.016) (layer B.Cu) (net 17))
 (segment (start 184.571 76.541) (end 184.444 76.668) (width 1.016) (layer B.Cu) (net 13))
 (segment (start 184.444 76.668) (end 184.444 77.201) (width 1.016) (layer B.Cu) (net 13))
 (segment (start 184.571 76.541) (end 184.571 75.271) (width 1.016) (layer B.Cu) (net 13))
 (segment (start 184.571 75.271) (end 187.071 72.771) (width 1.016) (layer B.Cu) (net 13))
 (segment (start 187.071 72.771) (end 189.611 72.771) (width 1.016) (layer B.Cu) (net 13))
 (segment (start 164.211 80.391) (end 181.991 80.391) (width 1.016) (layer B.Cu) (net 13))
 (segment (start 181.991 80.391) (end 184.571 77.811) (width 1.016) (layer B.Cu) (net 13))
 (segment (start 184.571 77.811) (end 184.571 76.541) (width 1.016) (layer B.Cu) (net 13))
 (segment (start 123.571 65.151) (end 123.571 68.961) (width 1.016) (layer B.Cu) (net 12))
 (segment (start 157.861 72.771) (end 155.321 72.771) (width 1.016) (layer B.Cu) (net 12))
 (segment (start 155.321 72.771) (end 147.701 65.151) (width 1.016) (layer B.Cu) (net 12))
 (segment (start 147.701 65.151) (end 123.571 65.151) (width 1.016) (layer B.Cu) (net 12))
 (segment (start 157.861 72.771) (end 160.401 72.771) (width 1.016) (layer B.Cu) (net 12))
 (segment (start 160.401 72.771) (end 164.211 68.961) (width 1.016) (layer B.Cu) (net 12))
 (segment (start 164.211 68.961) (end 164.211 67.691) (width 1.016) (layer B.Cu) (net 12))
 (segment (start 164.211 67.691) (end 164.211 66.421) (width 1.016) (layer B.Cu) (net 12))
 (segment (start 164.211 66.421) (end 165.481 65.151) (width 1.016) (layer B.Cu) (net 12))
 (segment (start 165.481 65.151) (end 176.911 65.151) (width 1.016) (layer B.Cu) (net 12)))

